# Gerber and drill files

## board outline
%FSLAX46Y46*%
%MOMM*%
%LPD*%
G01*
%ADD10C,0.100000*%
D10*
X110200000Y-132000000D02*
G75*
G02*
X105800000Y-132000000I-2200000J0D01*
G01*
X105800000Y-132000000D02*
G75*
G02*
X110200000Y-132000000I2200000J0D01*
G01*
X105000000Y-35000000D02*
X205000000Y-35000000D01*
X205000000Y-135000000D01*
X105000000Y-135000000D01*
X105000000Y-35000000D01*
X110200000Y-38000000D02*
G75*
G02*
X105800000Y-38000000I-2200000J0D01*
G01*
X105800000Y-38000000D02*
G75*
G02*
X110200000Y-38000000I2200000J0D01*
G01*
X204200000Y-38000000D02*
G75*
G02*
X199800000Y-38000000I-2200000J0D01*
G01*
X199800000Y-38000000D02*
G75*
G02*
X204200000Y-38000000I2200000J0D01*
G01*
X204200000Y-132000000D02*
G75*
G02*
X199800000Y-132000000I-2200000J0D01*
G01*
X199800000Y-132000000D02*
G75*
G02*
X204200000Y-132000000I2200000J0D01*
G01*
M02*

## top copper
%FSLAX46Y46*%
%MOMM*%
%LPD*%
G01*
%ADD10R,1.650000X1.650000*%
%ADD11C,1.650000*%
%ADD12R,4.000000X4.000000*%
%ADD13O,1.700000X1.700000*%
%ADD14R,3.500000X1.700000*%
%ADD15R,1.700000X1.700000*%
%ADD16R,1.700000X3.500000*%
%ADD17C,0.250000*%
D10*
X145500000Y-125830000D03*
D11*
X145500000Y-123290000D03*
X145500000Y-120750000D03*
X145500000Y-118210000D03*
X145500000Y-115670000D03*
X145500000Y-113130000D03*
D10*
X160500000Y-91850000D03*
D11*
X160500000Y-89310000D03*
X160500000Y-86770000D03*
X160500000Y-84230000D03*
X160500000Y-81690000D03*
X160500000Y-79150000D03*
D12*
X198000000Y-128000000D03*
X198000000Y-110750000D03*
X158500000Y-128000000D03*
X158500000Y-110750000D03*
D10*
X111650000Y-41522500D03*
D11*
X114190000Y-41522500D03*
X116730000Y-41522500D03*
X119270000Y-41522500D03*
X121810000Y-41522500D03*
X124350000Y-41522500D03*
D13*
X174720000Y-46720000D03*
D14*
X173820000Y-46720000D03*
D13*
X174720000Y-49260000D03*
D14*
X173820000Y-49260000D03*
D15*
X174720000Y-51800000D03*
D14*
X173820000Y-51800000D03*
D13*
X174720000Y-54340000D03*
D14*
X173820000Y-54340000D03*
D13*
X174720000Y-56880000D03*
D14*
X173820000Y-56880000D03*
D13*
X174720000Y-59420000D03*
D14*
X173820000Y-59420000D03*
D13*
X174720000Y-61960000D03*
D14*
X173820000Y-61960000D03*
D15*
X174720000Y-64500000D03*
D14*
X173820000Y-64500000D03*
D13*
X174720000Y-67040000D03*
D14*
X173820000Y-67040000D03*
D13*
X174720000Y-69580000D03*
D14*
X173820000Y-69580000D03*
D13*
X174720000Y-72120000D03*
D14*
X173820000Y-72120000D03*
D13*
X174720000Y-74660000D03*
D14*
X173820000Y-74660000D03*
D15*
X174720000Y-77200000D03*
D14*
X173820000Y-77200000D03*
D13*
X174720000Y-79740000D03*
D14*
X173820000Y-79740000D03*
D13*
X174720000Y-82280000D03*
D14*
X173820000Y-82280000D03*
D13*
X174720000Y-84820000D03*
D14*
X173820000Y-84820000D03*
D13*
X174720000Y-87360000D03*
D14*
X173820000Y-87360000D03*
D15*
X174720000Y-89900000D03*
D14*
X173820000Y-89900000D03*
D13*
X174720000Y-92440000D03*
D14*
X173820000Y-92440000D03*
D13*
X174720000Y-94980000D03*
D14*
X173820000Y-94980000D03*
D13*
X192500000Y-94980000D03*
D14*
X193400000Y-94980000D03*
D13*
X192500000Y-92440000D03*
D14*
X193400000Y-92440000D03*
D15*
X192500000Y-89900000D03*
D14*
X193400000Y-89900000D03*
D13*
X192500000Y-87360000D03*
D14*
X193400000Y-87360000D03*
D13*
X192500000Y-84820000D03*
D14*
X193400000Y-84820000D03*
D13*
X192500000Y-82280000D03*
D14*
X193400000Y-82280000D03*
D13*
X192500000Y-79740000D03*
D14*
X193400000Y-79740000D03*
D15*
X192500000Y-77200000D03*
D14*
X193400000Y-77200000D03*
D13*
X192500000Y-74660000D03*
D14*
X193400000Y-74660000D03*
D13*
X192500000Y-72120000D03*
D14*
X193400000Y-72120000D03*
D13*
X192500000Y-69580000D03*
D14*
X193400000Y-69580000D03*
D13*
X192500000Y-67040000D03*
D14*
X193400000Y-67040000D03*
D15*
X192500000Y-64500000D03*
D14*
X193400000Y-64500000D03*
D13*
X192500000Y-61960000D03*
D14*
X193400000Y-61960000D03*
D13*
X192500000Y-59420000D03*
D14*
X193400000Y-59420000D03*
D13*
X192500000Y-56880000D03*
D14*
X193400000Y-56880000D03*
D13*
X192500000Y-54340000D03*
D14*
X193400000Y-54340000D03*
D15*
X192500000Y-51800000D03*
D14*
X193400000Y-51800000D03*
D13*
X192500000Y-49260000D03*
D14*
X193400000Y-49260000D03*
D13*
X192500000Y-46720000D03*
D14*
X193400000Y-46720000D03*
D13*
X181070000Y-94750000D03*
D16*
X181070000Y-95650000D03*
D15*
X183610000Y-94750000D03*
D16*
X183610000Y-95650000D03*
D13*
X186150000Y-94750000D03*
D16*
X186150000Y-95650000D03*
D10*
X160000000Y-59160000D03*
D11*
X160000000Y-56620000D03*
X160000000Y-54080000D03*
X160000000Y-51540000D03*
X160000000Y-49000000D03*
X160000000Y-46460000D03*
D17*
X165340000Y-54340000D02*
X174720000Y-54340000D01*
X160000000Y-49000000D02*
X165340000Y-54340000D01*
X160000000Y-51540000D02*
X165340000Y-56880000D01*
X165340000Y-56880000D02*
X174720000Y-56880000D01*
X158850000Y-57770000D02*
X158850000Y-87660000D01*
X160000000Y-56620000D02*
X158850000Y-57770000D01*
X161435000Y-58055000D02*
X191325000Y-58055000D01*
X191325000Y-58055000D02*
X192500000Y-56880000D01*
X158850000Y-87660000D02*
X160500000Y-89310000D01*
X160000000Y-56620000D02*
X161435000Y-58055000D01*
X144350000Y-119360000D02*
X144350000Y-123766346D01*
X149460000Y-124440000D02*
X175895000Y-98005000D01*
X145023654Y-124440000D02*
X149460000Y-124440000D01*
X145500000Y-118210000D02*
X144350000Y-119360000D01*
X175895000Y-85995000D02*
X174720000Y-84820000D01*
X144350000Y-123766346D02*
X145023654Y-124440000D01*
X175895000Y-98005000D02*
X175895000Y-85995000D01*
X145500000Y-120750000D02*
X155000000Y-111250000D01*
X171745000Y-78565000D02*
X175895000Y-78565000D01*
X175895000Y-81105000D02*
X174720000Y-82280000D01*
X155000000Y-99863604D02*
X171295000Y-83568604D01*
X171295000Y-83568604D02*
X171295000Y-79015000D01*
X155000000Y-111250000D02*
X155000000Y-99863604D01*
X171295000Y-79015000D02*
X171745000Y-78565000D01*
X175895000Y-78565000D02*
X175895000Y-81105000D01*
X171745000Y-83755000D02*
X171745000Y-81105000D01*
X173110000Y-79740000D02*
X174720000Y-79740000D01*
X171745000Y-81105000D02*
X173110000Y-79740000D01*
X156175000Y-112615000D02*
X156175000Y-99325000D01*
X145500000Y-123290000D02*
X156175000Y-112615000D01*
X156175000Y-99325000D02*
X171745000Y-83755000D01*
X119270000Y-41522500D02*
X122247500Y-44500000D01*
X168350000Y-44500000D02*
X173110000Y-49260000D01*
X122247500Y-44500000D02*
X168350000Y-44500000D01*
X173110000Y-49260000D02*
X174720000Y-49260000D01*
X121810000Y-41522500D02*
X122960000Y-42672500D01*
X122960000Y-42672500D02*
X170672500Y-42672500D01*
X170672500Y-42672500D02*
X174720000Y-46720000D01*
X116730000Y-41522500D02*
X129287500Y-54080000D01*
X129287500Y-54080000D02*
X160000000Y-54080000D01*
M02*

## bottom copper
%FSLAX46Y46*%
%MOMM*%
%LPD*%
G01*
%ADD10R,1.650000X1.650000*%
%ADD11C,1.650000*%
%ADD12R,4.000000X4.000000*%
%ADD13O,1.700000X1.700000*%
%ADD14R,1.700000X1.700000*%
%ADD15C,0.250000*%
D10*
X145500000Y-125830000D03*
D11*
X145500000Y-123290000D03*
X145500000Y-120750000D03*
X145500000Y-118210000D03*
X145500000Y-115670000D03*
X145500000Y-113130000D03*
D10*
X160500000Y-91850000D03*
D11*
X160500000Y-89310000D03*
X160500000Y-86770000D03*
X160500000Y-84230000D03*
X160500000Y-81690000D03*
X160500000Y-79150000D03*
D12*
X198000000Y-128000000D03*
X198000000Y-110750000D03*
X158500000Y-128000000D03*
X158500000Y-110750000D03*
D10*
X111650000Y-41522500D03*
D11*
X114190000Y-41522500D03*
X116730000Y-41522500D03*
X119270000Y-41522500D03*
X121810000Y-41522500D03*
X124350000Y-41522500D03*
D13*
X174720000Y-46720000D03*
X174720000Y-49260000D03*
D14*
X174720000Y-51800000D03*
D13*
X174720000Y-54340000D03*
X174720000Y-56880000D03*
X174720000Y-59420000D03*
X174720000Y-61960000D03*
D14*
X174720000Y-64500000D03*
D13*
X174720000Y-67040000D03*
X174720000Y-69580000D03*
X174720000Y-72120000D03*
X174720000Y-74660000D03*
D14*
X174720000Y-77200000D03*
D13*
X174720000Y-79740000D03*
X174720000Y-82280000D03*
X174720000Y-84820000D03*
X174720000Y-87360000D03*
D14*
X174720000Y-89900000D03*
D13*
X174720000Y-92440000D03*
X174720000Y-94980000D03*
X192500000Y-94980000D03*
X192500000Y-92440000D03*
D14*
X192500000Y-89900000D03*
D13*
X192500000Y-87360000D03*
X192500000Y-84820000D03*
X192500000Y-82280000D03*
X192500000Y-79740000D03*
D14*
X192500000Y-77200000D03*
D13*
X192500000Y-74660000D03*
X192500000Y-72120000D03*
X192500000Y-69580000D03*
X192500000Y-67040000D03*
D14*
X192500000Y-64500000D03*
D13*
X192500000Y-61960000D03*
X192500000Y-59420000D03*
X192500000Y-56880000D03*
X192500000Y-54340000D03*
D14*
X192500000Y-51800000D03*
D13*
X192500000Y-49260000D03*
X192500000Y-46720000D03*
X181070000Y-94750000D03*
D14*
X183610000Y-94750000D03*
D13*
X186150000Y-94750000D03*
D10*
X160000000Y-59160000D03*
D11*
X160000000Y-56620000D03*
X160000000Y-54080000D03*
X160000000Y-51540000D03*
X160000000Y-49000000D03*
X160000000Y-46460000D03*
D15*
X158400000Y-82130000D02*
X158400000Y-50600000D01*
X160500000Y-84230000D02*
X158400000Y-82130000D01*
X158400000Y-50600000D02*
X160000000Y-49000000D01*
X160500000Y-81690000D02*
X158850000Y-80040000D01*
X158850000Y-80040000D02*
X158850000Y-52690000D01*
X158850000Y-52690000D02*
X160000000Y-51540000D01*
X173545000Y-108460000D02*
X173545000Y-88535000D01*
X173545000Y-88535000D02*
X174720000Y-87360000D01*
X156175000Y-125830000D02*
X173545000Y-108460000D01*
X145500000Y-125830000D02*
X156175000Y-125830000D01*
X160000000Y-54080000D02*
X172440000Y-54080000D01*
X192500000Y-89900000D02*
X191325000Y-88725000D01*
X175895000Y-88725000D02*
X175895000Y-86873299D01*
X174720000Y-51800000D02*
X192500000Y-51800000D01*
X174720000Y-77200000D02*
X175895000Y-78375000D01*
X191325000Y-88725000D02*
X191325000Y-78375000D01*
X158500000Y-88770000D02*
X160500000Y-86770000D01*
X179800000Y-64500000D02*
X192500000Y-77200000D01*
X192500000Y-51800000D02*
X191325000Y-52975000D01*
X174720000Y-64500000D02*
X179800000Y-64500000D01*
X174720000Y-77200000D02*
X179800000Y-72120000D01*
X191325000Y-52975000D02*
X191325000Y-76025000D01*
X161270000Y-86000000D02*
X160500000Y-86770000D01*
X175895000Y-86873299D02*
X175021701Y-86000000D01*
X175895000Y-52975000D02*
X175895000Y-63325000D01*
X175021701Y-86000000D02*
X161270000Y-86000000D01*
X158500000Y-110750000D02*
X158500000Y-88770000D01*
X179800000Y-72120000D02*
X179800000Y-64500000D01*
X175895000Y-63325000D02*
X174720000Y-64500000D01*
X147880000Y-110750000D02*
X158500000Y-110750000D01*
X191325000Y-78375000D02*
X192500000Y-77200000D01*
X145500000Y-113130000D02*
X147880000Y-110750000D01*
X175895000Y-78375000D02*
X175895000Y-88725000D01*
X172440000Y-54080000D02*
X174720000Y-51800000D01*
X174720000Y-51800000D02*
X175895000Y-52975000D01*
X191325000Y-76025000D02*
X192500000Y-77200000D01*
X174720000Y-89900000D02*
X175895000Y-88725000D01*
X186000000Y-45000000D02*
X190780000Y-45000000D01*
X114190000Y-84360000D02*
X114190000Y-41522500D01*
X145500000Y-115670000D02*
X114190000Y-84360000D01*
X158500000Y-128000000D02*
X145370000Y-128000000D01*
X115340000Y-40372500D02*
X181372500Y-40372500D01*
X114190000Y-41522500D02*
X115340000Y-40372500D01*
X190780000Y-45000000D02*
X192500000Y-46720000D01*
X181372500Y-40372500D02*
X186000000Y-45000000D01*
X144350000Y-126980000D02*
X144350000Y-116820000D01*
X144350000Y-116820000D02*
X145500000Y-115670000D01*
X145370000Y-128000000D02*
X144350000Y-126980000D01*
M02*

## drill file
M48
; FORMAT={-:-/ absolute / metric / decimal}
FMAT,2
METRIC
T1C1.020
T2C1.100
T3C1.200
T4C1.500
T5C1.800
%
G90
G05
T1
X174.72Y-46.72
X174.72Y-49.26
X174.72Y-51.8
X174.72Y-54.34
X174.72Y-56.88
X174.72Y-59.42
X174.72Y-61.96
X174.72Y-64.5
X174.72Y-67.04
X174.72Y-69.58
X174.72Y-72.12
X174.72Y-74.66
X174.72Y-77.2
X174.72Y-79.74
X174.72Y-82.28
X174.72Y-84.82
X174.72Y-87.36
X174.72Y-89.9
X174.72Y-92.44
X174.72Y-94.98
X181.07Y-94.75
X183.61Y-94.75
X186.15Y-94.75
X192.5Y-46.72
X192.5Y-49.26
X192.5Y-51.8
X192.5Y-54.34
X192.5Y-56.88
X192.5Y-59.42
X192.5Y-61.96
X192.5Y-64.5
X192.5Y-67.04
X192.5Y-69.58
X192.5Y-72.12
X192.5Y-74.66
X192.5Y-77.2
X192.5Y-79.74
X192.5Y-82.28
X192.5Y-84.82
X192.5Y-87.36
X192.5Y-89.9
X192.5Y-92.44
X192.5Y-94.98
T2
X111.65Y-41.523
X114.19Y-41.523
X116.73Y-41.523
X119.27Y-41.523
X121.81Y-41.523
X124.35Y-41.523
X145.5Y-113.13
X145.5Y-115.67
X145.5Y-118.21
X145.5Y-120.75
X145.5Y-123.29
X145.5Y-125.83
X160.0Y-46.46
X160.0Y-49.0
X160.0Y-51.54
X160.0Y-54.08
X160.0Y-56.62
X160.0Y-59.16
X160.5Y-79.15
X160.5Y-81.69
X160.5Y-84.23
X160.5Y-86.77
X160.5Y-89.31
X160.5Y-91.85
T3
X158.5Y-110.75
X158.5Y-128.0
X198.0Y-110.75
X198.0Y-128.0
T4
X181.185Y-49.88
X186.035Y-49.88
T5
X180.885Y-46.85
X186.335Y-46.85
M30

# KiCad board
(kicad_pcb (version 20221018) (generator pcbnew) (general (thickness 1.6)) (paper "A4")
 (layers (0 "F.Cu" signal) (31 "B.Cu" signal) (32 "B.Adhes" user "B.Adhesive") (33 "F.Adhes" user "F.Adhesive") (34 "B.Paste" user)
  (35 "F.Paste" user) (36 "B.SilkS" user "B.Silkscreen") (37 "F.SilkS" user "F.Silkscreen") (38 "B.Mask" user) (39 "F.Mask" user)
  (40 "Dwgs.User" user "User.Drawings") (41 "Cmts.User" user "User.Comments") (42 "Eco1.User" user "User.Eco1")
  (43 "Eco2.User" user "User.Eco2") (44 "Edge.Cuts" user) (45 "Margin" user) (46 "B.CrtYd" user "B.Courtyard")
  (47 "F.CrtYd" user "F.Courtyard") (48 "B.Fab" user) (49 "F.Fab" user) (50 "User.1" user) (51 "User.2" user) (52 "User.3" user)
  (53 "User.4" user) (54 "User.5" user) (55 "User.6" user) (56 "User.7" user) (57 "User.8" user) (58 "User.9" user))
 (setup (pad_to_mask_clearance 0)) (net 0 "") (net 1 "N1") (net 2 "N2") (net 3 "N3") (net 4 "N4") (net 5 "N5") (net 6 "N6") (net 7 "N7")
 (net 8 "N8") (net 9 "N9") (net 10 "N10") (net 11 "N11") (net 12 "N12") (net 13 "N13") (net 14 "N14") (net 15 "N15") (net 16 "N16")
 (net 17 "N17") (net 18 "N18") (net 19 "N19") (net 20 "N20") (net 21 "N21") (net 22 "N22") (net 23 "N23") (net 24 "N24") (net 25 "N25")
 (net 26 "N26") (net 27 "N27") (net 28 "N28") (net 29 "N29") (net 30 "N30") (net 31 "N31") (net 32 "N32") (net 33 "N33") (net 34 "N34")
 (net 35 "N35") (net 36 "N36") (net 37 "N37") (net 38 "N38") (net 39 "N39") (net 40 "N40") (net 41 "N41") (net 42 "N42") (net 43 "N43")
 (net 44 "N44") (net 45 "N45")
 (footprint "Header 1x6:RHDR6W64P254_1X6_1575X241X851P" (layer "F.Cu") (at 145.5 125.83 -90)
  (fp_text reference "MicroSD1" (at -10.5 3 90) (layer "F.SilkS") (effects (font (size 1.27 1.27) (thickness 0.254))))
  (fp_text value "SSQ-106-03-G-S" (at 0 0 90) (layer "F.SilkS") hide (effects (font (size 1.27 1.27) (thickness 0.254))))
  (pad "1" thru_hole rect (at 0 0 270) (size 1.65 1.65) (drill 1.1) (layers "*.Cu" "*.Mask") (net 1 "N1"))
  (pad "2" thru_hole circle (at -2.54 0 270) (size 1.65 1.65) (drill 1.1) (layers "*.Cu" "*.Mask") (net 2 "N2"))
  (pad "3" thru_hole circle (at -5.08 0 270) (size 1.65 1.65) (drill 1.1) (layers "*.Cu" "*.Mask") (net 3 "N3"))
  (pad "4" thru_hole circle (at -7.62 0 270) (size 1.65 1.65) (drill 1.1) (layers "*.Cu" "*.Mask") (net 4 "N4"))
  (pad "5" thru_hole circle (at -10.16 0 270) (size 1.65 1.65) (drill 1.1) (layers "*.Cu" "*.Mask") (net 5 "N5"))
  (pad "6" thru_hole circle (at -12.7 0 270) (size 1.65 1.65) (drill 1.1) (layers "*.Cu" "*.Mask") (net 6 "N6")))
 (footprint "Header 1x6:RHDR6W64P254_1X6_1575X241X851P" (layer "F.Cu") (at 160.5 91.85 -90)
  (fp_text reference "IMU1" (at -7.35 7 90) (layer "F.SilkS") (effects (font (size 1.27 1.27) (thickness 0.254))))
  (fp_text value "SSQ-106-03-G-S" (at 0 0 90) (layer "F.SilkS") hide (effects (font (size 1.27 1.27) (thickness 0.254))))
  (pad "1" thru_hole rect (at 0 0 270) (size 1.65 1.65) (drill 1.1) (layers "*.Cu" "*.Mask") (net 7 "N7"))
  (pad "2" thru_hole circle (at -2.54 0 270) (size 1.65 1.65) (drill 1.1) (layers "*.Cu" "*.Mask") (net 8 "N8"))
  (pad "3" thru_hole circle (at -5.08 0 270) (size 1.65 1.65) (drill 1.1) (layers "*.Cu" "*.Mask") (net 6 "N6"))
  (pad "4" thru_hole circle (at -7.62 0 270) (size 1.65 1.65) (drill 1.1) (layers "*.Cu" "*.Mask") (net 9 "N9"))
  (pad "5" thru_hole circle (at -10.16 0 270) (size 1.65 1.65) (drill 1.1) (layers "*.Cu" "*.Mask") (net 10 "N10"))
  (pad "6" thru_hole circle (at -12.7 0 270) (size 1.65 1.65) (drill 1.1) (layers "*.Cu" "*.Mask") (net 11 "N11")))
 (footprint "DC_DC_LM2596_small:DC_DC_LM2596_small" (layer "F.Cu") (at 178.25 119.375 180)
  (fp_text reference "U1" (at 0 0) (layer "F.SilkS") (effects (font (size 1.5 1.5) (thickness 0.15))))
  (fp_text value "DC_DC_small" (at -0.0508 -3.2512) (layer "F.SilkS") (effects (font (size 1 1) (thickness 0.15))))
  (pad "1" thru_hole rect (at -19.75 -8.625 180) (size 4 4) (drill 1.2) (layers "*.Cu" "*.Mask" "F.SilkS") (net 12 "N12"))
  (pad "2" thru_hole rect (at -19.75 8.625 180) (size 4 4) (drill 1.2) (layers "*.Cu" "*.Mask" "F.SilkS") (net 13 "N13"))
  (pad "3" thru_hole rect (at 19.75 -8.625 180) (size 4 4) (drill 1.2) (layers "*.Cu" "*.Mask" "F.SilkS") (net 5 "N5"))
  (pad "4" thru_hole rect (at 19.75 8.625 180) (size 4 4) (drill 1.2) (layers "*.Cu" "*.Mask" "F.SilkS") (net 6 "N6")))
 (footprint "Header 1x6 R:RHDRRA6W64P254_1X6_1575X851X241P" (layer "F.Cu") (at 111.65 41.5225 180)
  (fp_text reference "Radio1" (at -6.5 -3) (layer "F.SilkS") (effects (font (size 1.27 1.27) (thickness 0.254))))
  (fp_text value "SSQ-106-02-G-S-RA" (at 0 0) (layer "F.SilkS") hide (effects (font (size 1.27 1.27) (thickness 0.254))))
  (pad "1" thru_hole rect (at 0 0 180) (size 1.65 1.65) (drill 1.1) (layers "*.Cu" "*.Mask") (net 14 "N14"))
  (pad "2" thru_hole circle (at -2.54 0 180) (size 1.65 1.65) (drill 1.1) (layers "*.Cu" "*.Mask") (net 5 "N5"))
  (pad "3" thru_hole circle (at -5.08 0 180) (size 1.65 1.65) (drill 1.1) (layers "*.Cu" "*.Mask") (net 6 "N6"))
  (pad "4" thru_hole circle (at -7.62 0 180) (size 1.65 1.65) (drill 1.1) (layers "*.Cu" "*.Mask") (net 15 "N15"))
  (pad "5" thru_hole circle (at -10.16 0 180) (size 1.65 1.65) (drill 1.1) (layers "*.Cu" "*.Mask") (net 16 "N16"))
  (pad "6" thru_hole circle (at -12.7 0 180) (size 1.65 1.65) (drill 1.1) (layers "*.Cu" "*.Mask") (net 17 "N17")))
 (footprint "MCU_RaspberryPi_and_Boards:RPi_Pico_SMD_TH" (layer "F.Cu") (at 183.61 70.85)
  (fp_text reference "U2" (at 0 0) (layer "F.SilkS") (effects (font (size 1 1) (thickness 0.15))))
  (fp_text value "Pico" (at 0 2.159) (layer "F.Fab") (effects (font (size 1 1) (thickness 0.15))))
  (pad "" np_thru_hole oval (at -2.725 -24) (size 1.8 1.8) (drill 1.8) (layers "*.Cu" "*.Mask"))
  (pad "" np_thru_hole oval (at -2.425 -20.97) (size 1.5 1.5) (drill 1.5) (layers "*.Cu" "*.Mask"))
  (pad "" np_thru_hole oval (at 2.425 -20.97) (size 1.5 1.5) (drill 1.5) (layers "*.Cu" "*.Mask"))
  (pad "" np_thru_hole oval (at 2.725 -24) (size 1.8 1.8) (drill 1.8) (layers "*.Cu" "*.Mask"))
  (pad "1" thru_hole oval (at -8.89 -24.13) (size 1.7 1.7) (drill 1.02) (layers "*.Cu" "*.Mask") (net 16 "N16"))
  (pad "1" smd rect (at -8.89 -24.13) (size 3.5 1.7) (drill (offset -0.9 0)) (layers "F.Cu" "F.Mask") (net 16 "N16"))
  (pad "2" thru_hole oval (at -8.89 -21.59) (size 1.7 1.7) (drill 1.02) (layers "*.Cu" "*.Mask") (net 15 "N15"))
  (pad "2" smd rect (at -8.89 -21.59) (size 3.5 1.7) (drill (offset -0.9 0)) (layers "F.Cu" "F.Mask") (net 15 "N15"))
  (pad "3" thru_hole rect (at -8.89 -19.05) (size 1.7 1.7) (drill 1.02) (layers "*.Cu" "*.Mask") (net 6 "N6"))
  (pad "3" smd rect (at -8.89 -19.05) (size 3.5 1.7) (drill (offset -0.9 0)) (layers "F.Cu" "F.Mask") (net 6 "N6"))
  (pad "4" thru_hole oval (at -8.89 -16.51) (size 1.7 1.7) (drill 1.02) (layers "*.Cu" "*.Mask") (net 9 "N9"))
  (pad "4" smd rect (at -8.89 -16.51) (size 3.5 1.7) (drill (offset -0.9 0)) (layers "F.Cu" "F.Mask") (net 9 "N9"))
  (pad "5" thru_hole oval (at -8.89 -13.97) (size 1.7 1.7) (drill 1.02) (layers "*.Cu" "*.Mask") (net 10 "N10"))
  (pad "5" smd rect (at -8.89 -13.97) (size 3.5 1.7) (drill (offset -0.9 0)) (layers "F.Cu" "F.Mask") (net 10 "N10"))
  (pad "6" thru_hole oval (at -8.89 -11.43) (size 1.7 1.7) (drill 1.02) (layers "*.Cu" "*.Mask") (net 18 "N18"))
  (pad "6" smd rect (at -8.89 -11.43) (size 3.5 1.7) (drill (offset -0.9 0)) (layers "F.Cu" "F.Mask") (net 18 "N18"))
  (pad "7" thru_hole oval (at -8.89 -8.89) (size 1.7 1.7) (drill 1.02) (layers "*.Cu" "*.Mask") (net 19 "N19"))
  (pad "7" smd rect (at -8.89 -8.89) (size 3.5 1.7) (drill (offset -0.9 0)) (layers "F.Cu" "F.Mask") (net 19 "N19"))
  (pad "8" thru_hole rect (at -8.89 -6.35) (size 1.7 1.7) (drill 1.02) (layers "*.Cu" "*.Mask") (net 6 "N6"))
  (pad "8" smd rect (at -8.89 -6.35) (size 3.5 1.7) (drill (offset -0.9 0)) (layers "F.Cu" "F.Mask") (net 6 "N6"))
  (pad "9" thru_hole oval (at -8.89 -3.81) (size 1.7 1.7) (drill 1.02) (layers "*.Cu" "*.Mask") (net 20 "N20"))
  (pad "9" smd rect (at -8.89 -3.81) (size 3.5 1.7) (drill (offset -0.9 0)) (layers "F.Cu" "F.Mask") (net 20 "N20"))
  (pad "10" thru_hole oval (at -8.89 -1.27) (size 1.7 1.7) (drill 1.02) (layers "*.Cu" "*.Mask") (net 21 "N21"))
  (pad "10" smd rect (at -8.89 -1.27) (size 3.5 1.7) (drill (offset -0.9 0)) (layers "F.Cu" "F.Mask") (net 21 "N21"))
  (pad "11" thru_hole oval (at -8.89 1.27) (size 1.7 1.7) (drill 1.02) (layers "*.Cu" "*.Mask") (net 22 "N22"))
  (pad "11" smd rect (at -8.89 1.27) (size 3.5 1.7) (drill (offset -0.9 0)) (layers "F.Cu" "F.Mask") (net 22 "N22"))
  (pad "12" thru_hole oval (at -8.89 3.81) (size 1.7 1.7) (drill 1.02) (layers "*.Cu" "*.Mask") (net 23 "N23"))
  (pad "12" smd rect (at -8.89 3.81) (size 3.5 1.7) (drill (offset -0.9 0)) (layers "F.Cu" "F.Mask") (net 23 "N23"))
  (pad "13" thru_hole rect (at -8.89 6.35) (size 1.7 1.7) (drill 1.02) (layers "*.Cu" "*.Mask") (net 6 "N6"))
  (pad "13" smd rect (at -8.89 6.35) (size 3.5 1.7) (drill (offset -0.9 0)) (layers "F.Cu" "F.Mask") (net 6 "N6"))
  (pad "14" thru_hole oval (at -8.89 8.89) (size 1.7 1.7) (drill 1.02) (layers "*.Cu" "*.Mask") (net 2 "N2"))
  (pad "14" smd rect (at -8.89 8.89) (size 3.5 1.7) (drill (offset -0.9 0)) (layers "F.Cu" "F.Mask") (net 2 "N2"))
  (pad "15" thru_hole oval (at -8.89 11.43) (size 1.7 1.7) (drill 1.02) (layers "*.Cu" "*.Mask") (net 3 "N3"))
  (pad "15" smd rect (at -8.89 11.43) (size 3.5 1.7) (drill (offset -0.9 0)) (layers "F.Cu" "F.Mask") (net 3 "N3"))
  (pad "16" thru_hole oval (at -8.89 13.97) (size 1.7 1.7) (drill 1.02) (layers "*.Cu" "*.Mask") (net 4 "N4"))
  (pad "16" smd rect (at -8.89 13.97) (size 3.5 1.7) (drill (offset -0.9 0)) (layers "F.Cu" "F.Mask") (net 4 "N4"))
  (pad "17" thru_hole oval (at -8.89 16.51) (size 1.7 1.7) (drill 1.02) (layers "*.Cu" "*.Mask") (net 1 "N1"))
  (pad "17" smd rect (at -8.89 16.51) (size 3.5 1.7) (drill (offset -0.9 0)) (layers "F.Cu" "F.Mask") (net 1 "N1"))
  (pad "18" thru_hole rect (at -8.89 19.05) (size 1.7 1.7) (drill 1.02) (layers "*.Cu" "*.Mask") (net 6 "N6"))
  (pad "18" smd rect (at -8.89 19.05) (size 3.5 1.7) (drill (offset -0.9 0)) (layers "F.Cu" "F.Mask") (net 6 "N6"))
  (pad "19" thru_hole oval (at -8.89 21.59) (size 1.7 1.7) (drill 1.02) (layers "*.Cu" "*.Mask") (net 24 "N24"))
  (pad "19" smd rect (at -8.89 21.59) (size 3.5 1.7) (drill (offset -0.9 0)) (layers "F.Cu" "F.Mask") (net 24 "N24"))
  (pad "20" thru_hole oval (at -8.89 24.13) (size 1.7 1.7) (drill 1.02) (layers "*.Cu" "*.Mask") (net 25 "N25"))
  (pad "20" smd rect (at -8.89 24.13) (size 3.5 1.7) (drill (offset -0.9 0)) (layers "F.Cu" "F.Mask") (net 25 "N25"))
  (pad "21" thru_hole oval (at 8.89 24.13) (size 1.7 1.7) (drill 1.02) (layers "*.Cu" "*.Mask") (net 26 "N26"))
  (pad "21" smd rect (at 8.89 24.13) (size 3.5 1.7) (drill (offset 0.9 0)) (layers "F.Cu" "F.Mask") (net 26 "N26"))
  (pad "22" thru_hole oval (at 8.89 21.59) (size 1.7 1.7) (drill 1.02) (layers "*.Cu" "*.Mask") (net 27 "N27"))
  (pad "22" smd rect (at 8.89 21.59) (size 3.5 1.7) (drill (offset 0.9 0)) (layers "F.Cu" "F.Mask") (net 27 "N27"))
  (pad "23" thru_hole rect (at 8.89 19.05) (size 1.7 1.7) (drill 1.02) (layers "*.Cu" "*.Mask") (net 6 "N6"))
  (pad "23" smd rect (at 8.89 19.05) (size 3.5 1.7) (drill (offset 0.9 0)) (layers "F.Cu" "F.Mask") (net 6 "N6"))
  (pad "24" thru_hole oval (at 8.89 16.51) (size 1.7 1.7) (drill 1.02) (layers "*.Cu" "*.Mask") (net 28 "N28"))
  (pad "24" smd rect (at 8.89 16.51) (size 3.5 1.7) (drill (offset 0.9 0)) (layers "F.Cu" "F.Mask") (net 28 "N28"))
  (pad "25" thru_hole oval (at 8.89 13.97) (size 1.7 1.7) (drill 1.02) (layers "*.Cu" "*.Mask") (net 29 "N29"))
  (pad "25" smd rect (at 8.89 13.97) (size 3.5 1.7) (drill (offset 0.9 0)) (layers "F.Cu" "F.Mask") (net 29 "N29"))
  (pad "26" thru_hole oval (at 8.89 11.43) (size 1.7 1.7) (drill 1.02) (layers "*.Cu" "*.Mask") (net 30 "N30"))
  (pad "26" smd rect (at 8.89 11.43) (size 3.5 1.7) (drill (offset 0.9 0)) (layers "F.Cu" "F.Mask") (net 30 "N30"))
  (pad "27" thru_hole oval (at 8.89 8.89) (size 1.7 1.7) (drill 1.02) (layers "*.Cu" "*.Mask") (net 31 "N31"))
  (pad "27" smd rect (at 8.89 8.89) (size 3.5 1.7) (drill (offset 0.9 0)) (layers "F.Cu" "F.Mask") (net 31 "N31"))
  (pad "28" thru_hole rect (at 8.89 6.35) (size 1.7 1.7) (drill 1.02) (layers "*.Cu" "*.Mask") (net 6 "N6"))
  (pad "28" smd rect (at 8.89 6.35) (size 3.5 1.7) (drill (offset 0.9 0)) (layers "F.Cu" "F.Mask") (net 6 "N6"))
  (pad "29" thru_hole oval (at 8.89 3.81) (size 1.7 1.7) (drill 1.02) (layers "*.Cu" "*.Mask") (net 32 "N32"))
  (pad "29" smd rect (at 8.89 3.81) (size 3.5 1.7) (drill (offset 0.9 0)) (layers "F.Cu" "F.Mask") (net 32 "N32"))
  (pad "30" thru_hole oval (at 8.89 1.27) (size 1.7 1.7) (drill 1.02) (layers "*.Cu" "*.Mask") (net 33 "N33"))
  (pad "30" smd rect (at 8.89 1.27) (size 3.5 1.7) (drill (offset 0.9 0)) (layers "F.Cu" "F.Mask") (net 33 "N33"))
  (pad "31" thru_hole oval (at 8.89 -1.27) (size 1.7 1.7) (drill 1.02) (layers "*.Cu" "*.Mask") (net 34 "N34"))
  (pad "31" smd rect (at 8.89 -1.27) (size 3.5 1.7) (drill (offset 0.9 0)) (layers "F.Cu" "F.Mask") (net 34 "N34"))
  (pad "32" thru_hole oval (at 8.89 -3.81) (size 1.7 1.7) (drill 1.02) (layers "*.Cu" "*.Mask") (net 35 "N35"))
  (pad "32" smd rect (at 8.89 -3.81) (size 3.5 1.7) (drill (offset 0.9 0)) (layers "F.Cu" "F.Mask") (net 35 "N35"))
  (pad "33" thru_hole rect (at 8.89 -6.35) (size 1.7 1.7) (drill 1.02) (layers "*.Cu" "*.Mask") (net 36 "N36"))
  (pad "33" smd rect (at 8.89 -6.35) (size 3.5 1.7) (drill (offset 0.9 0)) (layers "F.Cu" "F.Mask") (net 36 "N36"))
  (pad "34" thru_hole oval (at 8.89 -8.89) (size 1.7 1.7) (drill 1.02) (layers "*.Cu" "*.Mask") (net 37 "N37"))
  (pad "34" smd rect (at 8.89 -8.89) (size 3.5 1.7) (drill (offset 0.9 0)) (layers "F.Cu" "F.Mask") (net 37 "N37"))
  (pad "35" thru_hole oval (at 8.89 -11.43) (size 1.7 1.7) (drill 1.02) (layers "*.Cu" "*.Mask") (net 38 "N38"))
  (pad "35" smd rect (at 8.89 -11.43) (size 3.5 1.7) (drill (offset 0.9 0)) (layers "F.Cu" "F.Mask") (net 38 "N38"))
  (pad "36" thru_hole oval (at 8.89 -13.97) (size 1.7 1.7) (drill 1.02) (layers "*.Cu" "*.Mask") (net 8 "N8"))
  (pad "36" smd rect (at 8.89 -13.97) (size 3.5 1.7) (drill (offset 0.9 0)) (layers "F.Cu" "F.Mask") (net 8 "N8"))
  (pad "37" thru_hole oval (at 8.89 -16.51) (size 1.7 1.7) (drill 1.02) (layers "*.Cu" "*.Mask") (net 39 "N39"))
  (pad "37" smd rect (at 8.89 -16.51) (size 3.5 1.7) (drill (offset 0.9 0)) (layers "F.Cu" "F.Mask") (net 39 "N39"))
  (pad "38" thru_hole rect (at 8.89 -19.05) (size 1.7 1.7) (drill 1.02) (layers "*.Cu" "*.Mask") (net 6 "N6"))
  (pad "38" smd rect (at 8.89 -19.05) (size 3.5 1.7) (drill (offset 0.9 0)) (layers "F.Cu" "F.Mask") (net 6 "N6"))
  (pad "39" thru_hole oval (at 8.89 -21.59) (size 1.7 1.7) (drill 1.02) (layers "*.Cu" "*.Mask") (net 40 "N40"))
  (pad "39" smd rect (at 8.89 -21.59) (size 3.5 1.7) (drill (offset 0.9 0)) (layers "F.Cu" "F.Mask") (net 40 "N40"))
  (pad "40" thru_hole oval (at 8.89 -24.13) (size 1.7 1.7) (drill 1.02) (layers "*.Cu" "*.Mask") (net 5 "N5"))
  (pad "40" smd rect (at 8.89 -24.13) (size 3.5 1.7) (drill (offset 0.9 0)) (layers "F.Cu" "F.Mask") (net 5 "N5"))
  (pad "41" thru_hole oval (at -2.54 23.9) (size 1.7 1.7) (drill 1.02) (layers "*.Cu" "*.Mask") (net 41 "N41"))
  (pad "41" smd rect (at -2.54 23.9 90) (size 3.5 1.7) (drill (offset -0.9 0)) (layers "F.Cu" "F.Mask") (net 41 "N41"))
  (pad "42" thru_hole rect (at 0 23.9) (size 1.7 1.7) (drill 1.02) (layers "*.Cu" "*.Mask") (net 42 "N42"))
  (pad "42" smd rect (at 0 23.9 90) (size 3.5 1.7) (drill (offset -0.9 0)) (layers "F.Cu" "F.Mask") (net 42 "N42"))
  (pad "43" thru_hole oval (at 2.54 23.9) (size 1.7 1.7) (drill 1.02) (layers "*.Cu" "*.Mask") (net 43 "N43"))
  (pad "43" smd rect (at 2.54 23.9 90) (size 3.5 1.7) (drill (offset -0.9 0)) (layers "F.Cu" "F.Mask") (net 43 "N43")))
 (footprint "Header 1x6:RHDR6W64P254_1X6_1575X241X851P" (layer "F.Cu") (at 160 59.16 -90)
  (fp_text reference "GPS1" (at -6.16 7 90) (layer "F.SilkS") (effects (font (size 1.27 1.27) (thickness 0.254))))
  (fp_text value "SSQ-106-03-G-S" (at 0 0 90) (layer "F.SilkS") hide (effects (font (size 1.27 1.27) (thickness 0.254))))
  (pad "1" thru_hole rect (at 0 0 270) (size 1.65 1.65) (drill 1.1) (layers "*.Cu" "*.Mask") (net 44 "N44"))
  (pad "2" thru_hole circle (at -2.54 0 270) (size 1.65 1.65) (drill 1.1) (layers "*.Cu" "*.Mask") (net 8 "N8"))
  (pad "3" thru_hole circle (at -5.08 0 270) (size 1.65 1.65) (drill 1.1) (layers "*.Cu" "*.Mask") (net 6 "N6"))
  (pad "4" thru_hole circle (at -7.62 0 270) (size 1.65 1.65) (drill 1.1) (layers "*.Cu" "*.Mask") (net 10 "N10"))
  (pad "5" thru_hole circle (at -10.16 0 270) (size 1.65 1.65) (drill 1.1) (layers "*.Cu" "*.Mask") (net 9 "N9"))
  (pad "6" thru_hole circle (at -12.7 0 270) (size 1.65 1.65) (drill 1.1) (layers "*.Cu" "*.Mask") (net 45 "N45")))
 (gr_circle (center 108 132) (end 110.2 132) (stroke (width 0.1) (type default)) (fill none) (layer "Edge.Cuts"))
 (gr_rect (start 105 35) (end 205 135) (stroke (width 0.1) (type default)) (fill none) (layer "Edge.Cuts"))
 (gr_circle (center 108 38) (end 110.2 38) (stroke (width 0.1) (type default)) (fill none) (layer "Edge.Cuts"))
 (gr_circle (center 202 38) (end 204.2 38) (stroke (width 0.1) (type default)) (fill none) (layer "Edge.Cuts"))
 (gr_circle (center 202 132) (end 204.2 132) (stroke (width 0.1) (type default)) (fill none) (layer "Edge.Cuts"))
 (segment (start 165.34 54.34) (end 174.72 54.34) (width 0.25) (layer "F.Cu") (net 9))
 (segment (start 160 49) (end 165.34 54.34) (width 0.25) (layer "F.Cu") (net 9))
 (segment (start 158.4 82.13) (end 158.4 50.6) (width 0.25) (layer "B.Cu") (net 9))
 (segment (start 160.5 84.23) (end 158.4 82.13) (width 0.25) (layer "B.Cu") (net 9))
 (segment (start 158.4 50.6) (end 160 49) (width 0.25) (layer "B.Cu") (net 9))
 (segment (start 160 51.54) (end 165.34 56.88) (width 0.25) (layer "F.Cu") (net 10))
 (segment (start 165.34 56.88) (end 174.72 56.88) (width 0.25) (layer "F.Cu") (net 10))
 (segment (start 160.5 81.69) (end 158.85 80.04) (width 0.25) (layer "B.Cu") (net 10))
 (segment (start 158.85 80.04) (end 158.85 52.69) (width 0.25) (layer "B.Cu") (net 10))
 (segment (start 158.85 52.69) (end 160 51.54) (width 0.25) (layer "B.Cu") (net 10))
 (segment (start 158.85 57.77) (end 158.85 87.66) (width 0.25) (layer "F.Cu") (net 8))
 (segment (start 160 56.62) (end 158.85 57.77) (width 0.25) (layer "F.Cu") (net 8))
 (segment (start 161.435 58.055) (end 191.325 58.055) (width 0.25) (layer "F.Cu") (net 8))
 (segment (start 191.325 58.055) (end 192.5 56.88) (width 0.25) (layer "F.Cu") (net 8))
 (segment (start 158.85 87.66) (end 160.5 89.31) (width 0.25) (layer "F.Cu") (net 8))
 (segment (start 160 56.62) (end 161.435 58.055) (width 0.25) (layer "F.Cu") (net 8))
 (segment (start 144.35 119.36) (end 144.35 123.766346) (width 0.25) (layer "F.Cu") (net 4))
 (segment (start 149.46 124.44) (end 175.895 98.005) (width 0.25) (layer "F.Cu") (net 4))
 (segment (start 145.023654 124.44) (end 149.46 124.44) (width 0.25) (layer "F.Cu") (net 4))
 (segment (start 145.5 118.21) (end 144.35 119.36) (width 0.25) (layer "F.Cu") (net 4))
 (segment (start 175.895 85.995) (end 174.72 84.82) (width 0.25) (layer "F.Cu") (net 4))
 (segment (start 144.35 123.766346) (end 145.023654 124.44) (width 0.25) (layer "F.Cu") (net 4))
 (segment (start 175.895 98.005) (end 175.895 85.995) (width 0.25) (layer "F.Cu") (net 4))
 (segment (start 145.5 120.75) (end 155 111.25) (width 0.25) (layer "F.Cu") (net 3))
 (segment (start 171.745 78.565) (end 175.895 78.565) (width 0.25) (layer "F.Cu") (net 3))
 (segment (start 175.895 81.105) (end 174.72 82.28) (width 0.25) (layer "F.Cu") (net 3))
 (segment (start 155 99.863604) (end 171.295 83.568604) (width 0.25) (layer "F.Cu") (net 3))
 (segment (start 171.295 83.568604) (end 171.295 79.015) (width 0.25) (layer "F.Cu") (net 3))
 (segment (start 155 111.25) (end 155 99.863604) (width 0.25) (layer "F.Cu") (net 3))
 (segment (start 171.295 79.015) (end 171.745 78.565) (width 0.25) (layer "F.Cu") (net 3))
 (segment (start 175.895 78.565) (end 175.895 81.105) (width 0.25) (layer "F.Cu") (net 3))
 (segment (start 171.745 83.755) (end 171.745 81.105) (width 0.25) (layer "F.Cu") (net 2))
 (segment (start 173.11 79.74) (end 174.72 79.74) (width 0.25) (layer "F.Cu") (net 2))
 (segment (start 171.745 81.105) (end 173.11 79.74) (width 0.25) (layer "F.Cu") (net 2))
 (segment (start 156.175 112.615) (end 156.175 99.325) (width 0.25) (layer "F.Cu") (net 2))
 (segment (start 145.5 123.29) (end 156.175 112.615) (width 0.25) (layer "F.Cu") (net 2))
 (segment (start 156.175 99.325) (end 171.745 83.755) (width 0.25) (layer "F.Cu") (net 2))
 (segment (start 173.545 108.46) (end 173.545 88.535) (width 0.25) (layer "B.Cu") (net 1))
 (segment (start 173.545 88.535) (end 174.72 87.36) (width 0.25) (layer "B.Cu") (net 1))
 (segment (start 156.175 125.83) (end 173.545 108.46) (width 0.25) (layer "B.Cu") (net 1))
 (segment (start 145.5 125.83) (end 156.175 125.83) (width 0.25) (layer "B.Cu") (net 1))
 (segment (start 119.27 41.5225) (end 122.2475 44.5) (width 0.25) (layer "F.Cu") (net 15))
 (segment (start 168.35 44.5) (end 173.11 49.26) (width 0.25) (layer "F.Cu") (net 15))
 (segment (start 122.2475 44.5) (end 168.35 44.5) (width 0.25) (layer "F.Cu") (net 15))
 (segment (start 173.11 49.26) (end 174.72 49.26) (width 0.25) (layer "F.Cu") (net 15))
 (segment (start 121.81 41.5225) (end 122.96 42.6725) (width 0.25) (layer "F.Cu") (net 16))
 (segment (start 122.96 42.6725) (end 170.6725 42.6725) (width 0.25) (layer "F.Cu") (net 16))
 (segment (start 170.6725 42.6725) (end 174.72 46.72) (width 0.25) (layer "F.Cu") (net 16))
 (segment (start 116.73 41.5225) (end 129.2875 54.08) (width 0.25) (layer "F.Cu") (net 6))
 (segment (start 129.2875 54.08) (end 160 54.08) (width 0.25) (layer "F.Cu") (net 6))
 (segment (start 160 54.08) (end 172.44 54.08) (width 0.25) (layer "B.Cu") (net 6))
 (segment (start 192.5 89.9) (end 191.325 88.725) (width 0.25) (layer "B.Cu") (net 6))
 (segment (start 175.895 88.725) (end 175.895 86.873299) (width 0.25) (layer "B.Cu") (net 6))
 (segment (start 174.72 51.8) (end 192.5 51.8) (width 0.25) (layer "B.Cu") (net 6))
 (segment (start 174.72 77.2) (end 175.895 78.375) (width 0.25) (layer "B.Cu") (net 6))
 (segment (start 191.325 88.725) (end 191.325 78.375) (width 0.25) (layer "B.Cu") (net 6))
 (segment (start 158.5 88.77) (end 160.5 86.77) (width 0.25) (layer "B.Cu") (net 6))
 (segment (start 179.8 64.5) (end 192.5 77.2) (width 0.25) (layer "B.Cu") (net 6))
 (segment (start 192.5 51.8) (end 191.325 52.975) (width 0.25) (layer "B.Cu") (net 6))
 (segment (start 174.72 64.5) (end 179.8 64.5) (width 0.25) (layer "B.Cu") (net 6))
 (segment (start 174.72 77.2) (end 179.8 72.12) (width 0.25) (layer "B.Cu") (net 6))
 (segment (start 191.325 52.975) (end 191.325 76.025) (width 0.25) (layer "B.Cu") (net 6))
 (segment (start 161.27 86) (end 160.5 86.77) (width 0.25) (layer "B.Cu") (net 6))
 (segment (start 175.895 86.873299) (end 175.021701 86) (width 0.25) (layer "B.Cu") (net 6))
 (segment (start 175.895 52.975) (end 175.895 63.325) (width 0.25) (layer "B.Cu") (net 6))
 (segment (start 175.021701 86) (end 161.27 86) (width 0.25) (layer "B.Cu") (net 6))
 (segment (start 158.5 110.75) (end 158.5 88.77) (width 0.25) (layer "B.Cu") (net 6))
 (segment (start 179.8 72.12) (end 179.8 64.5) (width 0.25) (layer "B.Cu") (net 6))
 (segment (start 175.895 63.325) (end 174.72 64.5) (width 0.25) (layer "B.Cu") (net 6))
 (segment (start 147.88 110.75) (end 158.5 110.75) (width 0.25) (layer "B.Cu") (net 6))
 (segment (start 191.325 78.375) (end 192.5 77.2) (width 0.25) (layer "B.Cu") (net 6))
 (segment (start 145.5 113.13) (end 147.88 110.75) (width 0.25) (layer "B.Cu") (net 6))
 (segment (start 175.895 78.375) (end 175.895 88.725) (width 0.25) (layer "B.Cu") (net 6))
 (segment (start 172.44 54.08) (end 174.72 51.8) (width 0.25) (layer "B.Cu") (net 6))
 (segment (start 174.72 51.8) (end 175.895 52.975) (width 0.25) (layer "B.Cu") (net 6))
 (segment (start 191.325 76.025) (end 192.5 77.2) (width 0.25) (layer "B.Cu") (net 6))
 (segment (start 174.72 89.9) (end 175.895 88.725) (width 0.25) (layer "B.Cu") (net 6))
 (segment (start 186 45) (end 190.78 45) (width 0.25) (layer "B.Cu") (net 5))
 (segment (start 114.19 84.36) (end 114.19 41.5225) (width 0.25) (layer "B.Cu") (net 5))
 (segment (start 145.5 115.67) (end 114.19 84.36) (width 0.25) (layer "B.Cu") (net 5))
 (segment (start 158.5 128) (end 145.37 128) (width 0.25) (layer "B.Cu") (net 5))
 (segment (start 115.34 40.3725) (end 181.3725 40.3725) (width 0.25) (layer "B.Cu") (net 5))
 (segment (start 114.19 41.5225) (end 115.34 40.3725) (width 0.25) (layer "B.Cu") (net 5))
 (segment (start 190.78 45) (end 192.5 46.72) (width 0.25) (layer "B.Cu") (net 5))
 (segment (start 181.3725 40.3725) (end 186 45) (width 0.25) (layer "B.Cu") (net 5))
 (segment (start 144.35 126.98) (end 144.35 116.82) (width 0.25) (layer "B.Cu") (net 5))
 (segment (start 144.35 116.82) (end 145.5 115.67) (width 0.25) (layer "B.Cu") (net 5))
 (segment (start 145.37 128) (end 144.35 126.98) (width 0.25) (layer "B.Cu") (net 5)))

